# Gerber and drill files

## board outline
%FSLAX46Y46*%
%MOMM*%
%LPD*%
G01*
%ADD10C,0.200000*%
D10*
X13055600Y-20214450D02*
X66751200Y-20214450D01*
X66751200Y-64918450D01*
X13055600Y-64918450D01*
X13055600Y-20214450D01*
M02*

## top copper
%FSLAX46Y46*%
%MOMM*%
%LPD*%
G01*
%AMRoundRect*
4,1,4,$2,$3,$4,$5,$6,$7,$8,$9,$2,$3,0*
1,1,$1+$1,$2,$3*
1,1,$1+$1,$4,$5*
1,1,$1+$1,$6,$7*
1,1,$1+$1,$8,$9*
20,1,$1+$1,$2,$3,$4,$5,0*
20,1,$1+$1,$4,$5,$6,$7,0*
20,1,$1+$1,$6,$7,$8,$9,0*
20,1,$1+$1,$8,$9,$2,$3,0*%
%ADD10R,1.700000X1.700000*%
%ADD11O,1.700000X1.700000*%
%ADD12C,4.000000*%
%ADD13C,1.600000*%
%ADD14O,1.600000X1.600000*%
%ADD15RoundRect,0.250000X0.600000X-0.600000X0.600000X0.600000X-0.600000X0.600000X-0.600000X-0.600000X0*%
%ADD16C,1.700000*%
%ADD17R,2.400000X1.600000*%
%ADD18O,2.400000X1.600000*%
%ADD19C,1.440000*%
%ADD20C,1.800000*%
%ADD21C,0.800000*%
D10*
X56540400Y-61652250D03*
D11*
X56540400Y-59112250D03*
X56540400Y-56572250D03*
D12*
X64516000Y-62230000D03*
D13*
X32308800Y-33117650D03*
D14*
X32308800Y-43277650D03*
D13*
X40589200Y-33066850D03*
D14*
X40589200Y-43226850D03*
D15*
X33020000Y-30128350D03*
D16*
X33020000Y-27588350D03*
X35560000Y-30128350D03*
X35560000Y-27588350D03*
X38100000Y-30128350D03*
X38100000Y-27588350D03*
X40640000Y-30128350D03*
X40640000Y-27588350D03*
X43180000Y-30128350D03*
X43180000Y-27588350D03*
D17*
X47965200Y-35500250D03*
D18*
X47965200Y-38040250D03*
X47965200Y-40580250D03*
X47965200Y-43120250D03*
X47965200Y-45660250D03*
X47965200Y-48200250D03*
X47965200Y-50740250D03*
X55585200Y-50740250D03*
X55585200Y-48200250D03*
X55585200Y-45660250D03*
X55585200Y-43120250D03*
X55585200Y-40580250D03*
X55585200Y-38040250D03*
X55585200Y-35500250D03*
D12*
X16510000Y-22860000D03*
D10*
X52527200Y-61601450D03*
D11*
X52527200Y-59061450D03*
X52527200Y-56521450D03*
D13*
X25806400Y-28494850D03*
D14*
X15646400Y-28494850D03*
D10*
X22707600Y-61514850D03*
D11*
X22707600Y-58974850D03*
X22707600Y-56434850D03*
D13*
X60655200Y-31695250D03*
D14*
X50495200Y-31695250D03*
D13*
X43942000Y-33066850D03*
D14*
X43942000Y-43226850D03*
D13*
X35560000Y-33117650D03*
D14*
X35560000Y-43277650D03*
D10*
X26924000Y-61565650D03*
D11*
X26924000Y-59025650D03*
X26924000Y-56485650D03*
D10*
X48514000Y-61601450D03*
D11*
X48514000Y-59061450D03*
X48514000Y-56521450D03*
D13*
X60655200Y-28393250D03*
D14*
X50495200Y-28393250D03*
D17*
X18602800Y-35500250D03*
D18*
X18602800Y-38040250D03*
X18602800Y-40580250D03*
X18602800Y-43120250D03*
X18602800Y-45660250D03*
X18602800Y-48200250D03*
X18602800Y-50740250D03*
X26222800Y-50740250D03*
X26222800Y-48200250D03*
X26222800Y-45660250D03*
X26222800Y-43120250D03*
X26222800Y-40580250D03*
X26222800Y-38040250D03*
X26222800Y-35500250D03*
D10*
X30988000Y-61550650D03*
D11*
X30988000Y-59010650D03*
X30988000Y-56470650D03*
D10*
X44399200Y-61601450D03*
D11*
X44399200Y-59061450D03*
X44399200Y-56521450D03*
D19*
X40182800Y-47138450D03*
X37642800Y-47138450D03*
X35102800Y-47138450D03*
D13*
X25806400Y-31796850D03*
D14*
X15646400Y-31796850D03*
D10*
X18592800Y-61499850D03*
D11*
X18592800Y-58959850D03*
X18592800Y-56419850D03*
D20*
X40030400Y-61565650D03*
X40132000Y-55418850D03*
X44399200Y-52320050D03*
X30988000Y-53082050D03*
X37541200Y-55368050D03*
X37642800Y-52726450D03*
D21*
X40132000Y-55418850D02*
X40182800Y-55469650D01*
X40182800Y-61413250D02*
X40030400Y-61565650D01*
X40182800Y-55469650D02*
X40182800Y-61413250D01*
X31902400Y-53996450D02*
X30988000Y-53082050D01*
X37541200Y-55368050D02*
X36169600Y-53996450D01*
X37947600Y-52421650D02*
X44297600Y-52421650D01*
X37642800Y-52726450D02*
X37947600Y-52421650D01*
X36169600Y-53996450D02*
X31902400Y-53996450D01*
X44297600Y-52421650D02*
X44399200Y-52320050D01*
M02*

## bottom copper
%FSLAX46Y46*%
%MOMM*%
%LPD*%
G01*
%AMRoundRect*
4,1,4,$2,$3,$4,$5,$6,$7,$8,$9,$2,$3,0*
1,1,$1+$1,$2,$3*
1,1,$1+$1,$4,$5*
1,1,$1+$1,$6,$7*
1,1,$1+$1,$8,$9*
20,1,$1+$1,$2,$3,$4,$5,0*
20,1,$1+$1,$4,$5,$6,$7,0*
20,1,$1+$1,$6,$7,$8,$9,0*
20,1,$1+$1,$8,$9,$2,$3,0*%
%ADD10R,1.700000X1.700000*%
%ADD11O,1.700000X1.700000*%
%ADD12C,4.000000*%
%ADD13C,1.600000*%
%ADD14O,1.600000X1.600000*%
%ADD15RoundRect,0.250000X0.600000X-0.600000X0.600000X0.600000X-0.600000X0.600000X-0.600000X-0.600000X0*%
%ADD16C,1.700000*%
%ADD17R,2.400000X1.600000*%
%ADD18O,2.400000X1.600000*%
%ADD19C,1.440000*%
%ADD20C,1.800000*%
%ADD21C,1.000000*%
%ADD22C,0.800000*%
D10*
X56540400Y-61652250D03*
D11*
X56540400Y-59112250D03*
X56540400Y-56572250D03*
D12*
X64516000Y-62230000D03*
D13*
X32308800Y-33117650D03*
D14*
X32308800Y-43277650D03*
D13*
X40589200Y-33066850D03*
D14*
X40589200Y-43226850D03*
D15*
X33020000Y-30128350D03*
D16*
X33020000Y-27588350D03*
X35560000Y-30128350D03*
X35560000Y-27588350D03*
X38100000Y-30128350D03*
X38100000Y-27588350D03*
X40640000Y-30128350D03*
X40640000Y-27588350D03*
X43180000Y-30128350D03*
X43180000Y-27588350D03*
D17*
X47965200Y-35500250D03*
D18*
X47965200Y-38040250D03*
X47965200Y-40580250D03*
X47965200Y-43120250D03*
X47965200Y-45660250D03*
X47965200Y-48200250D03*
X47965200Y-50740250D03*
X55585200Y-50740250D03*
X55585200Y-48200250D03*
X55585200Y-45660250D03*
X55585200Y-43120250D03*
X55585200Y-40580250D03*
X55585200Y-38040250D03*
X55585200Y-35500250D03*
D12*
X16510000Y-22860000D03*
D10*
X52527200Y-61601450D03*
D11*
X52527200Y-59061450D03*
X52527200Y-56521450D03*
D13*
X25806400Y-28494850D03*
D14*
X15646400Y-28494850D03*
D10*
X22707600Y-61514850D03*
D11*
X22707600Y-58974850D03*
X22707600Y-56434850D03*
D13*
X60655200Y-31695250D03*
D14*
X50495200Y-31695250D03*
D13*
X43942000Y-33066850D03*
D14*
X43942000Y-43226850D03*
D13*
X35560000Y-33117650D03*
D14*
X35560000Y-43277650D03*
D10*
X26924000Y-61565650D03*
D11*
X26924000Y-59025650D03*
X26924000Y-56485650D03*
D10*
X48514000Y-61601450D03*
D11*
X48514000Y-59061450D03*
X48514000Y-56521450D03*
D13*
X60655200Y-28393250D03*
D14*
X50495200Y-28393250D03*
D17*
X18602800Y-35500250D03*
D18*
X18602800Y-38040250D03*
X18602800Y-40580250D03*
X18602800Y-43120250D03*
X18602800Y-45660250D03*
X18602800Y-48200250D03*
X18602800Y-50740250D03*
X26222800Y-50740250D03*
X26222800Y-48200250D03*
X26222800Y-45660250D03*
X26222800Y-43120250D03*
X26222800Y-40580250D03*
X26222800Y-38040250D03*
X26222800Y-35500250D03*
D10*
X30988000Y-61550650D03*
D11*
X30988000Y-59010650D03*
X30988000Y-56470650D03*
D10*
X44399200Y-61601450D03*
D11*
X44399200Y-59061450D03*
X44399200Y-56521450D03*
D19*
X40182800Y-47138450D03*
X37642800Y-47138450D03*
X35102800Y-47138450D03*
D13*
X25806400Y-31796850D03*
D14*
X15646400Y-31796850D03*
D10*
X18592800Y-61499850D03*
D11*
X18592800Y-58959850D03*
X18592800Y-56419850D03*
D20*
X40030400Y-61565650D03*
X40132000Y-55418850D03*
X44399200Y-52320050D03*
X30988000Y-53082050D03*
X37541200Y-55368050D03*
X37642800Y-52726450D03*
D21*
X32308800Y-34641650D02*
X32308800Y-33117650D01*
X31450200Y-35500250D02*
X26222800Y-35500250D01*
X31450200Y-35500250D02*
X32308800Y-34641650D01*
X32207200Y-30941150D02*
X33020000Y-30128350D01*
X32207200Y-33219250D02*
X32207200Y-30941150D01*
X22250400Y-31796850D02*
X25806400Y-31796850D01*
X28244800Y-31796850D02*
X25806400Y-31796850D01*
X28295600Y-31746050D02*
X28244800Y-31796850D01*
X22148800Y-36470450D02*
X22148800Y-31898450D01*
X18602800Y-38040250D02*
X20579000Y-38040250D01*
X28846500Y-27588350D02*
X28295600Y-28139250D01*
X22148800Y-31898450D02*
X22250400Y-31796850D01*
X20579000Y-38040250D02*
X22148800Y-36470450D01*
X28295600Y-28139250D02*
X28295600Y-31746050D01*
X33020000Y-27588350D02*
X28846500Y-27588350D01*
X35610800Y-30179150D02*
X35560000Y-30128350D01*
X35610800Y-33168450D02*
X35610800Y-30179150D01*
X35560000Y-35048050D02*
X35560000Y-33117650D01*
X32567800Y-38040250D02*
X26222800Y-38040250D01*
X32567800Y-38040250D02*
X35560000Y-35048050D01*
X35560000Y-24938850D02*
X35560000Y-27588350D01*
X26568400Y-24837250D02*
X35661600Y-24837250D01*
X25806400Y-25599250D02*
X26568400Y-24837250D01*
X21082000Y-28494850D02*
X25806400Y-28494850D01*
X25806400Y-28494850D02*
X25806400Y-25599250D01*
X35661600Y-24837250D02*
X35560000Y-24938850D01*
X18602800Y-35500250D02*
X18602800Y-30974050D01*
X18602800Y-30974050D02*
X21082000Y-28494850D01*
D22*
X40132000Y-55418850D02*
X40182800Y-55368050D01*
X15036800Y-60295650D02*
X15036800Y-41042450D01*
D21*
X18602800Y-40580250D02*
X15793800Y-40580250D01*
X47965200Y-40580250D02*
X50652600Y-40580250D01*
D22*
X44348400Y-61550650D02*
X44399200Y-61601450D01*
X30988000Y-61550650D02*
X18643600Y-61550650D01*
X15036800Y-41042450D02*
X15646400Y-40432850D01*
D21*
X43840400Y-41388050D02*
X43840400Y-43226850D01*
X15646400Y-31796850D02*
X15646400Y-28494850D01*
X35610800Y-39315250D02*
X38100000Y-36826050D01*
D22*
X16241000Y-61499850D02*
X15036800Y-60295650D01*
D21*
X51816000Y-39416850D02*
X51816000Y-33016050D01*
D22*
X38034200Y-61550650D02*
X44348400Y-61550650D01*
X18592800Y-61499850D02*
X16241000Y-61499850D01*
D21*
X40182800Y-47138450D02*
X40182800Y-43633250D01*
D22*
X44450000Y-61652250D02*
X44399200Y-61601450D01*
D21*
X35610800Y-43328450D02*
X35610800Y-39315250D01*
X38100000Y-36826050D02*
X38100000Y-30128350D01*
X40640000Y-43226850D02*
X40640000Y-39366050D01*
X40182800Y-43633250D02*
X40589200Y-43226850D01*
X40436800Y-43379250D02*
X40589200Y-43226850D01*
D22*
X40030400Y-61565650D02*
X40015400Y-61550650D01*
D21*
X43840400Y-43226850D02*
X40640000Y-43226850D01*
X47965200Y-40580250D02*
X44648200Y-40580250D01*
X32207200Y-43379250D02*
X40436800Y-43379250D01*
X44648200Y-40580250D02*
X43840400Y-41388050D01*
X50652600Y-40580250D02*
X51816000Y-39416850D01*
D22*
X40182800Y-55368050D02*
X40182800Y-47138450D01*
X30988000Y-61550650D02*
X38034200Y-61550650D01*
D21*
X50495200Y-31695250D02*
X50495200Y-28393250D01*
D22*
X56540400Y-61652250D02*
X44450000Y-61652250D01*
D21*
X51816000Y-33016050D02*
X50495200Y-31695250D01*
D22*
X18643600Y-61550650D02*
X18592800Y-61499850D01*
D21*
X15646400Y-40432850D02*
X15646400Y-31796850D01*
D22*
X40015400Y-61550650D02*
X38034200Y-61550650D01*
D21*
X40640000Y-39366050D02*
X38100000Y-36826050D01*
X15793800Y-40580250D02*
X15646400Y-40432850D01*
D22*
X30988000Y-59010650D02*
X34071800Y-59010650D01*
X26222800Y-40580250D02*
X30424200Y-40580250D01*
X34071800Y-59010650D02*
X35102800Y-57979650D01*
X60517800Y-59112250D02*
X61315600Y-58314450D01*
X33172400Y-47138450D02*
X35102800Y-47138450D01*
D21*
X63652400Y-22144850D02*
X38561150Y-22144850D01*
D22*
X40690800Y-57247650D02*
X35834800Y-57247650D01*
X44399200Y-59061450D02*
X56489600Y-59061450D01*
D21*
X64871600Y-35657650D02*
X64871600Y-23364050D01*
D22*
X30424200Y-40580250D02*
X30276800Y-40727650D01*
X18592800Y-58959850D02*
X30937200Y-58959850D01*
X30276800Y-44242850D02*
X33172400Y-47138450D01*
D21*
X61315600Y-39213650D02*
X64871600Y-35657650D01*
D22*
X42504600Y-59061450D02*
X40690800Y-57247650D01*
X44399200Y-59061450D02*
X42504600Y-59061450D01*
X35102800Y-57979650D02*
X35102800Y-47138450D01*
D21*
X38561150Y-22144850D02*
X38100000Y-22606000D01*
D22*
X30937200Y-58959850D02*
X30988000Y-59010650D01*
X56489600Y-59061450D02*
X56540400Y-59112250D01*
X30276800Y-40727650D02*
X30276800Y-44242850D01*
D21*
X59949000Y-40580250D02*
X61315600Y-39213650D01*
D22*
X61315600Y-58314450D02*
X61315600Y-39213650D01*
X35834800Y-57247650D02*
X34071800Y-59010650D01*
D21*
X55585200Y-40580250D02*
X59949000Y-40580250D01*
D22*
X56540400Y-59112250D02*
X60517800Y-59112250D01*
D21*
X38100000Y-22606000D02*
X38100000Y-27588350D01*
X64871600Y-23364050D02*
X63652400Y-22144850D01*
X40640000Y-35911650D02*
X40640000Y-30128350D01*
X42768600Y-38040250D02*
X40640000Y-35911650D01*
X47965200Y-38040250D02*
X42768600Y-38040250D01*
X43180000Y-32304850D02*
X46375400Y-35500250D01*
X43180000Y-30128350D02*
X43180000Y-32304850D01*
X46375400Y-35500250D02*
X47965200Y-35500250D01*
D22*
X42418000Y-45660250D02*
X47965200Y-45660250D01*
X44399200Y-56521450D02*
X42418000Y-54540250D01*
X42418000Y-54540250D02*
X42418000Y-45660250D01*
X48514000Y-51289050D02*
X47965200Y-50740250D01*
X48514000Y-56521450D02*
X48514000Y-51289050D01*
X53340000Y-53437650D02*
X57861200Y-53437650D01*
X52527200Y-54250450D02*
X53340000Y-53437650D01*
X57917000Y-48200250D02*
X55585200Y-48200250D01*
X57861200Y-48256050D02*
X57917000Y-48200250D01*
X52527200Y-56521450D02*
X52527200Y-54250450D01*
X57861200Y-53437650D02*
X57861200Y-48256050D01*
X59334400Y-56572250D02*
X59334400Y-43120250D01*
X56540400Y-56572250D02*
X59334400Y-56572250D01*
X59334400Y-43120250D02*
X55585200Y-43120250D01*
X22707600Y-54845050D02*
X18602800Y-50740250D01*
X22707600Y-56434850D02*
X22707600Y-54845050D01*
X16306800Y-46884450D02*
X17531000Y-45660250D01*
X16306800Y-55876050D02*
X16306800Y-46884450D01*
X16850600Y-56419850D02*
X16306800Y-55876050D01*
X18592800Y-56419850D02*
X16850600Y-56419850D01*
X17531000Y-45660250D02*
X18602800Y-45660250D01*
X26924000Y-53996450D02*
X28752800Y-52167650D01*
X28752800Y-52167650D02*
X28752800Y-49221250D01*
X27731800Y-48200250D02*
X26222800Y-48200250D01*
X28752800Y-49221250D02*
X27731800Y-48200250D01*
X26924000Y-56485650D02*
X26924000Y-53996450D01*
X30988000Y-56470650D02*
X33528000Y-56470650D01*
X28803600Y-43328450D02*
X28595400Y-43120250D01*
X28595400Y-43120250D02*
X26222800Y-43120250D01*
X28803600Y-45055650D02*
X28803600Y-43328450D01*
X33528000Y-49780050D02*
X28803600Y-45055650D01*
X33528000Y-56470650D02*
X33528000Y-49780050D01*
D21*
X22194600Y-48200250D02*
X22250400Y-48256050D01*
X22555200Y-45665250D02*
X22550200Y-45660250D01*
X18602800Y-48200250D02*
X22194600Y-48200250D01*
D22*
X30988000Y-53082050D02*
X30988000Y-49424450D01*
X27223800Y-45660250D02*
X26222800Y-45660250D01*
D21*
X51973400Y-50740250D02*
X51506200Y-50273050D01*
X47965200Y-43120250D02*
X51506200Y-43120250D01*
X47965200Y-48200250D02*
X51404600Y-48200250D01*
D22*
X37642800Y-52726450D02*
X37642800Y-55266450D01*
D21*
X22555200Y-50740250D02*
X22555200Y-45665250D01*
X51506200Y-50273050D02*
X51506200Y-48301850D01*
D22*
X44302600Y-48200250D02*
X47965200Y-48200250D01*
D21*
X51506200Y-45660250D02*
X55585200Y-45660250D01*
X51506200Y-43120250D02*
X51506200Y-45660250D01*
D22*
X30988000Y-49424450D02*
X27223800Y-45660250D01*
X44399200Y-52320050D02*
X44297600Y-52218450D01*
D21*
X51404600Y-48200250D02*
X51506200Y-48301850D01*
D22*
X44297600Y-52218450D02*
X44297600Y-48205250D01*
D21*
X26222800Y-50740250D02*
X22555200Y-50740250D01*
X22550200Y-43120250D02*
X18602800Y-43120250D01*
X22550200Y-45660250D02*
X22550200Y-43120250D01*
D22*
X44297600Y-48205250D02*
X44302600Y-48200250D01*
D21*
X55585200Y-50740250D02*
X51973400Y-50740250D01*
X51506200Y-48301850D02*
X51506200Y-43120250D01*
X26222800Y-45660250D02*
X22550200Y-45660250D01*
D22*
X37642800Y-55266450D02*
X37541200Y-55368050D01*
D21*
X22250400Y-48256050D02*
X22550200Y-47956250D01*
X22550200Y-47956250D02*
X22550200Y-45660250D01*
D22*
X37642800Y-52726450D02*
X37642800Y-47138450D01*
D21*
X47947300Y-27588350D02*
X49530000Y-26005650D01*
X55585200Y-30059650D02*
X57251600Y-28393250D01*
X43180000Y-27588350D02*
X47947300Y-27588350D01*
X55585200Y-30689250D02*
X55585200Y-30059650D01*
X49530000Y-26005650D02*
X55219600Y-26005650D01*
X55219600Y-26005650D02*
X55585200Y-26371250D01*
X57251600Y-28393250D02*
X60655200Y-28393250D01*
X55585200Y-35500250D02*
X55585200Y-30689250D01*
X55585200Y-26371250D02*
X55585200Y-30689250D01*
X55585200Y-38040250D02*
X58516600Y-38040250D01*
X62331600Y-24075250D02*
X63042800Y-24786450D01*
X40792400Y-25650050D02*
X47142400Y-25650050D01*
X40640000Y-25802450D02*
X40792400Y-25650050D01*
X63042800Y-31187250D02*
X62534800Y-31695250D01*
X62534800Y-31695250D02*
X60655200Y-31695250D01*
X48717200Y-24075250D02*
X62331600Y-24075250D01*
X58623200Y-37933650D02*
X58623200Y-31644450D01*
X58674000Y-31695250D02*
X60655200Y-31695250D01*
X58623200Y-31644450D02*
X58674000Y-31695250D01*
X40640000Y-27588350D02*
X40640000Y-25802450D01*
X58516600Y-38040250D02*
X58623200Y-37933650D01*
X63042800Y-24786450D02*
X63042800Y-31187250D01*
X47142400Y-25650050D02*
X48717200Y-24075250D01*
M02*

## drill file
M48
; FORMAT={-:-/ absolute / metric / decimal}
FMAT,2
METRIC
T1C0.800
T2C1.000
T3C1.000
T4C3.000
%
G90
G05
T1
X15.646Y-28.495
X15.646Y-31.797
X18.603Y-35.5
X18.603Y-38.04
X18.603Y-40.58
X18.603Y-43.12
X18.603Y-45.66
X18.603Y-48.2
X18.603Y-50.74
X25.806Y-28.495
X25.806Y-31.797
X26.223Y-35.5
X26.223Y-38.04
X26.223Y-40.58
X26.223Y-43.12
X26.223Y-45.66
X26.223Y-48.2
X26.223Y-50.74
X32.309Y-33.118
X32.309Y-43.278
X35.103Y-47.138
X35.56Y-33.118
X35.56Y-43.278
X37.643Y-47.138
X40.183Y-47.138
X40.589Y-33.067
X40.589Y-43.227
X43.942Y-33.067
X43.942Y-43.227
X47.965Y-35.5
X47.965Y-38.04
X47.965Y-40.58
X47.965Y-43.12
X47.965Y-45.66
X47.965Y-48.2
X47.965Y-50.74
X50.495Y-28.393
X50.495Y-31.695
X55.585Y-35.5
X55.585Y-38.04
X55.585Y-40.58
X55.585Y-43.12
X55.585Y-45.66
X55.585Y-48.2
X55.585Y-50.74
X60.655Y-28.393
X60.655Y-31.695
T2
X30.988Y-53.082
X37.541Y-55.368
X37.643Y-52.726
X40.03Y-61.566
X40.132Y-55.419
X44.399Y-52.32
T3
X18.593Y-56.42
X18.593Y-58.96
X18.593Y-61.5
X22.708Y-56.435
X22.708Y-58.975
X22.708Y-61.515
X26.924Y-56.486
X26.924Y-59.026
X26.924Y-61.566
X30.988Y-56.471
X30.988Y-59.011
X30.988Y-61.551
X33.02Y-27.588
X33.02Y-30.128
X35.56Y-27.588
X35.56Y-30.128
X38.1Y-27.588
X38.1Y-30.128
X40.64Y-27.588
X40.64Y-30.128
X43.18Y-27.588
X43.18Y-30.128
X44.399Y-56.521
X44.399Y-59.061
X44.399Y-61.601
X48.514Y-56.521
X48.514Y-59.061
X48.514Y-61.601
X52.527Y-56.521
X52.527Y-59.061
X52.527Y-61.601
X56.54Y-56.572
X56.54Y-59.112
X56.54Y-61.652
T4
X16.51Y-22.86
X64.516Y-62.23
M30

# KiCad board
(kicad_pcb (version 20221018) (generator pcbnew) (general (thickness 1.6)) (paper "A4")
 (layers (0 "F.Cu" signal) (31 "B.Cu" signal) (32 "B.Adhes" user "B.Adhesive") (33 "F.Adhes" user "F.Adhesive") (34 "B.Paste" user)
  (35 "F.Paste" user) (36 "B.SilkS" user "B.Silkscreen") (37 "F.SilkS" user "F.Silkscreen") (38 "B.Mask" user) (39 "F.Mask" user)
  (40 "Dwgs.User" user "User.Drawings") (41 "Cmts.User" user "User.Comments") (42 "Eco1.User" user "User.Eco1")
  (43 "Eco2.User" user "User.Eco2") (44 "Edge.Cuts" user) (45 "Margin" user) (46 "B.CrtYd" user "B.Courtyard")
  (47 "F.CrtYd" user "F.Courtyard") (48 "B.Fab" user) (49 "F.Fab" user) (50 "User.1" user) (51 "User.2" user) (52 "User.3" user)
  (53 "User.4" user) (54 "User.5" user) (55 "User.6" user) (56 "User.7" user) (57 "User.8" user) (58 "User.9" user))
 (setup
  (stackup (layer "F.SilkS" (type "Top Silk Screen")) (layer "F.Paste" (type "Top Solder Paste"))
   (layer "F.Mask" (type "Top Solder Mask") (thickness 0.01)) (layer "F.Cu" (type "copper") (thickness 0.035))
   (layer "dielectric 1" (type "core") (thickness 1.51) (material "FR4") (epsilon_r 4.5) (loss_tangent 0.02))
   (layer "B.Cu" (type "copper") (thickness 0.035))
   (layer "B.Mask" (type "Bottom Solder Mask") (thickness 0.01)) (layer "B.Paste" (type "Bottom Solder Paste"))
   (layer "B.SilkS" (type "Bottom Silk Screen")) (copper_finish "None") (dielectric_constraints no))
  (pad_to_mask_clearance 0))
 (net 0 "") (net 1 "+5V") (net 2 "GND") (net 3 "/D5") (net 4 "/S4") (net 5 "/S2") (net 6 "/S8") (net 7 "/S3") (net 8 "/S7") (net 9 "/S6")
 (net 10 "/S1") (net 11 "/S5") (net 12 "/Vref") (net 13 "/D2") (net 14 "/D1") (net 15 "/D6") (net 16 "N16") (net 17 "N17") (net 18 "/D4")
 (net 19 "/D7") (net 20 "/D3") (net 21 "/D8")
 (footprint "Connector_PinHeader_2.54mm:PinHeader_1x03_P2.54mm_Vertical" (layer "F.Cu") (at 56.5404 61.65225 180)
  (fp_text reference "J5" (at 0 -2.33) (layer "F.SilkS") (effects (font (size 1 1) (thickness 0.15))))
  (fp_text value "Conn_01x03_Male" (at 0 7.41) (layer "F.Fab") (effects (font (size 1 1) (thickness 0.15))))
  (pad "1" thru_hole rect (at 0 0 180) (size 1.7 1.7) (drill 1) (layers "*.Cu" "*.Mask") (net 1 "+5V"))
  (pad "2" thru_hole oval (at 0 2.54 180) (size 1.7 1.7) (drill 1) (layers "*.Cu" "*.Mask") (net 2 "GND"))
  (pad "3" thru_hole oval (at 0 5.08 180) (size 1.7 1.7) (drill 1) (layers "*.Cu" "*.Mask") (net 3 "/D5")))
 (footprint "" (layer "F.Cu") (at 64.516 62.23)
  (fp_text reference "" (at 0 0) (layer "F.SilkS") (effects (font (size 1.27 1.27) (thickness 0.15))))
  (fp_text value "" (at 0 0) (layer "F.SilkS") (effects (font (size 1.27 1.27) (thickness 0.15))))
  (pad "1" thru_hole circle (at 0 0) (size 4 4) (drill 3) (layers "*.Cu" "*.Mask")))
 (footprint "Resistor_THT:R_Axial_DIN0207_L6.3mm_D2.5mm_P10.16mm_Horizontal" (layer "F.Cu") (at 32.3088 33.11765 -90)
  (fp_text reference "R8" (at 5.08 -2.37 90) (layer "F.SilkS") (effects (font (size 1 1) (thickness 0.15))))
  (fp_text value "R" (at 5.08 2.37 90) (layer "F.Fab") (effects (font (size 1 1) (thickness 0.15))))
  (pad "1" thru_hole circle (at 0 0 270) (size 1.6 1.6) (drill 0.8) (layers "*.Cu" "*.Mask") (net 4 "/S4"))
  (pad "2" thru_hole oval (at 10.16 0 270) (size 1.6 1.6) (drill 0.8) (layers "*.Cu" "*.Mask") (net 1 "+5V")))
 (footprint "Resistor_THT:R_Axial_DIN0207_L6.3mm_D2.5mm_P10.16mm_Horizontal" (layer "F.Cu") (at 40.5892 33.06685 -90)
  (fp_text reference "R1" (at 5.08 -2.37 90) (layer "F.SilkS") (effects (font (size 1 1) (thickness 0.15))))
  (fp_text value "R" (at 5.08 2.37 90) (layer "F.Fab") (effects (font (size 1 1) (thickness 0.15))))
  (pad "1" thru_hole circle (at 0 0 270) (size 1.6 1.6) (drill 0.8) (layers "*.Cu" "*.Mask") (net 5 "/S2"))
  (pad "2" thru_hole oval (at 10.16 0 270) (size 1.6 1.6) (drill 0.8) (layers "*.Cu" "*.Mask") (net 1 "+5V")))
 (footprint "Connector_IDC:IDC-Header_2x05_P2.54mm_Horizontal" (layer "F.Cu") (at 33.02 30.12835 90)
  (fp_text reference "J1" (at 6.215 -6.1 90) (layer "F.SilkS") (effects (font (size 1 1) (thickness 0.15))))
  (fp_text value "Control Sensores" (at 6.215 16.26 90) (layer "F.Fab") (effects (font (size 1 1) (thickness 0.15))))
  (pad "1" thru_hole roundrect (at 0 0 90) (size 1.7 1.7) (drill 1) (layers "*.Cu" "*.Mask") (roundrect_rratio 0.147059) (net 4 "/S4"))
  (pad "2" thru_hole circle (at 2.54 0 90) (size 1.7 1.7) (drill 1) (layers "*.Cu" "*.Mask") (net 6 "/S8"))
  (pad "3" thru_hole circle (at 0 2.54 90) (size 1.7 1.7) (drill 1) (layers "*.Cu" "*.Mask") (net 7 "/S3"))
  (pad "4" thru_hole circle (at 2.54 2.54 90) (size 1.7 1.7) (drill 1) (layers "*.Cu" "*.Mask") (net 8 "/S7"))
  (pad "5" thru_hole circle (at 0 5.08 90) (size 1.7 1.7) (drill 1) (layers "*.Cu" "*.Mask") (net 1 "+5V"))
  (pad "6" thru_hole circle (at 2.54 5.08 90) (size 1.7 1.7) (drill 1) (layers "*.Cu" "*.Mask") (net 2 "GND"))
  (pad "7" thru_hole circle (at 0 7.62 90) (size 1.7 1.7) (drill 1) (layers "*.Cu" "*.Mask") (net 5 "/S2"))
  (pad "8" thru_hole circle (at 2.54 7.62 90) (size 1.7 1.7) (drill 1) (layers "*.Cu" "*.Mask") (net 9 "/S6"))
  (pad "9" thru_hole circle (at 0 10.16 90) (size 1.7 1.7) (drill 1) (layers "*.Cu" "*.Mask") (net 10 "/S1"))
  (pad "10" thru_hole circle (at 2.54 10.16 90) (size 1.7 1.7) (drill 1) (layers "*.Cu" "*.Mask") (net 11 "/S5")))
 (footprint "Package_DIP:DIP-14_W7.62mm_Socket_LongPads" (layer "F.Cu") (at 47.9652 35.50025)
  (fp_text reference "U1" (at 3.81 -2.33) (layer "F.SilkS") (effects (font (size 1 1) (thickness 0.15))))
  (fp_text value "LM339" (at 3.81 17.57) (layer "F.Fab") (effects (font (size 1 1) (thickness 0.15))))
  (pad "1" thru_hole rect (at 0 0) (size 2.4 1.6) (drill 0.8) (layers "*.Cu" "*.Mask") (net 10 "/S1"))
  (pad "2" thru_hole oval (at 0 2.54) (size 2.4 1.6) (drill 0.8) (layers "*.Cu" "*.Mask") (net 5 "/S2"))
  (pad "3" thru_hole oval (at 0 5.08) (size 2.4 1.6) (drill 0.8) (layers "*.Cu" "*.Mask") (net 1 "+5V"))
  (pad "4" thru_hole oval (at 0 7.62) (size 2.4 1.6) (drill 0.8) (layers "*.Cu" "*.Mask") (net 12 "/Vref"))
  (pad "5" thru_hole oval (at 0 10.16) (size 2.4 1.6) (drill 0.8) (layers "*.Cu" "*.Mask") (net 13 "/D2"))
  (pad "6" thru_hole oval (at 0 12.7) (size 2.4 1.6) (drill 0.8) (layers "*.Cu" "*.Mask") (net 12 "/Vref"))
  (pad "7" thru_hole oval (at 0 15.24) (size 2.4 1.6) (drill 0.8) (layers "*.Cu" "*.Mask") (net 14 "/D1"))
  (pad "8" thru_hole oval (at 7.62 15.24) (size 2.4 1.6) (drill 0.8) (layers "*.Cu" "*.Mask") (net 12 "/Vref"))
  (pad "9" thru_hole oval (at 7.62 12.7) (size 2.4 1.6) (drill 0.8) (layers "*.Cu" "*.Mask") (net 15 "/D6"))
  (pad "10" thru_hole oval (at 7.62 10.16) (size 2.4 1.6) (drill 0.8) (layers "*.Cu" "*.Mask") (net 12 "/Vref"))
  (pad "11" thru_hole oval (at 7.62 7.62) (size 2.4 1.6) (drill 0.8) (layers "*.Cu" "*.Mask") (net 3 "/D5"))
  (pad "12" thru_hole oval (at 7.62 5.08) (size 2.4 1.6) (drill 0.8) (layers "*.Cu" "*.Mask") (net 2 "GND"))
  (pad "13" thru_hole oval (at 7.62 2.54) (size 2.4 1.6) (drill 0.8) (layers "*.Cu" "*.Mask") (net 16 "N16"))
  (pad "14" thru_hole oval (at 7.62 0) (size 2.4 1.6) (drill 0.8) (layers "*.Cu" "*.Mask") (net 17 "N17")))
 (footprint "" (layer "F.Cu") (at 16.51 22.86)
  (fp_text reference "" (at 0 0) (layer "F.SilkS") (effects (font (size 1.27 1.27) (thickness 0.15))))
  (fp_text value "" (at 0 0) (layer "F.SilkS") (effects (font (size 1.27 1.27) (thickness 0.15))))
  (pad "1" thru_hole circle (at 0 0) (size 4 4) (drill 3) (layers "*.Cu" "*.Mask")))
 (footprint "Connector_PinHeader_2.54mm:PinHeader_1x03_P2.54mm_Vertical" (layer "F.Cu") (at 52.5272 61.60145 180)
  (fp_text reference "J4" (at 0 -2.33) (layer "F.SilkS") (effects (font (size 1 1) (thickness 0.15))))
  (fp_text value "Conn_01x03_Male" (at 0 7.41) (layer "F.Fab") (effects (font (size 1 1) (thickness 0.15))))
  (pad "1" thru_hole rect (at 0 0 180) (size 1.7 1.7) (drill 1) (layers "*.Cu" "*.Mask") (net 1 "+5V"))
  (pad "2" thru_hole oval (at 0 2.54 180) (size 1.7 1.7) (drill 1) (layers "*.Cu" "*.Mask") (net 2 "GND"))
  (pad "3" thru_hole oval (at 0 5.08 180) (size 1.7 1.7) (drill 1) (layers "*.Cu" "*.Mask") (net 15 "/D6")))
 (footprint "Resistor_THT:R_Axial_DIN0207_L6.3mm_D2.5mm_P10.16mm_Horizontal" (layer "F.Cu") (at 25.8064 28.49485 180)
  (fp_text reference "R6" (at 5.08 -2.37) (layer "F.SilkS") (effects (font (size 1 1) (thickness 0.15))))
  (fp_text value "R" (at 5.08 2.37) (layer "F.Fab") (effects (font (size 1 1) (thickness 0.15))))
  (pad "1" thru_hole circle (at 0 0 180) (size 1.6 1.6) (drill 0.8) (layers "*.Cu" "*.Mask") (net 8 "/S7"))
  (pad "2" thru_hole oval (at 10.16 0 180) (size 1.6 1.6) (drill 0.8) (layers "*.Cu" "*.Mask") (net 1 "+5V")))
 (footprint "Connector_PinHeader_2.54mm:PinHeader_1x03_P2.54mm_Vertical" (layer "F.Cu") (at 22.7076 61.51485 180)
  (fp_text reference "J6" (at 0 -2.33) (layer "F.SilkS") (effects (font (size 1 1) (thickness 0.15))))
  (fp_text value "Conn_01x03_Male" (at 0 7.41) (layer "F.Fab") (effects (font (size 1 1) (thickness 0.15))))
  (pad "1" thru_hole rect (at 0 0 180) (size 1.7 1.7) (drill 1) (layers "*.Cu" "*.Mask") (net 1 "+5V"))
  (pad "2" thru_hole oval (at 0 2.54 180) (size 1.7 1.7) (drill 1) (layers "*.Cu" "*.Mask") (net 2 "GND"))
  (pad "3" thru_hole oval (at 0 5.08 180) (size 1.7 1.7) (drill 1) (layers "*.Cu" "*.Mask") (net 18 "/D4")))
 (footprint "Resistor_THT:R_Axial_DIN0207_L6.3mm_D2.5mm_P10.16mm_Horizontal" (layer "F.Cu") (at 60.6552 31.69525 180)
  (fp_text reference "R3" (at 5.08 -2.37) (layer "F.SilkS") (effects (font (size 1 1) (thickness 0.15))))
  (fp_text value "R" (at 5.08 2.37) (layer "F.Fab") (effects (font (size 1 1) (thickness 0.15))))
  (pad "1" thru_hole circle (at 0 0 180) (size 1.6 1.6) (drill 0.8) (layers "*.Cu" "*.Mask") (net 16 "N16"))
  (pad "2" thru_hole oval (at 10.16 0 180) (size 1.6 1.6) (drill 0.8) (layers "*.Cu" "*.Mask") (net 1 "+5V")))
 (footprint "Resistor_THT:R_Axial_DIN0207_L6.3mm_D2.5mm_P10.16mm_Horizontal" (layer "F.Cu") (at 43.942 33.06685 -90)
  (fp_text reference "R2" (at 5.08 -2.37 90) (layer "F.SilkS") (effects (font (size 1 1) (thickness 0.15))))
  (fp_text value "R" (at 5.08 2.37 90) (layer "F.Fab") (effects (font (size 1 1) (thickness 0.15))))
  (pad "1" thru_hole circle (at 0 0 270) (size 1.6 1.6) (drill 0.8) (layers "*.Cu" "*.Mask") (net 10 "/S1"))
  (pad "2" thru_hole oval (at 10.16 0 270) (size 1.6 1.6) (drill 0.8) (layers "*.Cu" "*.Mask") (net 1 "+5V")))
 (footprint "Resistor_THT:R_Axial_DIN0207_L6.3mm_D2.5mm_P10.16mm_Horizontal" (layer "F.Cu") (at 35.56 33.11765 -90)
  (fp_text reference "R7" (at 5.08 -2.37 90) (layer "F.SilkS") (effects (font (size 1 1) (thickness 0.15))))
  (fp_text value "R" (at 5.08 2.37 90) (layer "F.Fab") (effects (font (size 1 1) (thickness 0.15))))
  (pad "1" thru_hole circle (at 0 0 270) (size 1.6 1.6) (drill 0.8) (layers "*.Cu" "*.Mask") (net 7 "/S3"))
  (pad "2" thru_hole oval (at 10.16 0 270) (size 1.6 1.6) (drill 0.8) (layers "*.Cu" "*.Mask") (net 1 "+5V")))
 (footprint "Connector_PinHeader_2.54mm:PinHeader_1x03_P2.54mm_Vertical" (layer "F.Cu") (at 26.924 61.56565 180)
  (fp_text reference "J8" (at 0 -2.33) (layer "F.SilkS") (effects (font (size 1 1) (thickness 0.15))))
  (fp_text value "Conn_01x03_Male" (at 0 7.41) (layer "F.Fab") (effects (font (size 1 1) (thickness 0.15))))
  (pad "1" thru_hole rect (at 0 0 180) (size 1.7 1.7) (drill 1) (layers "*.Cu" "*.Mask") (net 1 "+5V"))
  (pad "2" thru_hole oval (at 0 2.54 180) (size 1.7 1.7) (drill 1) (layers "*.Cu" "*.Mask") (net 2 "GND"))
  (pad "3" thru_hole oval (at 0 5.08 180) (size 1.7 1.7) (drill 1) (layers "*.Cu" "*.Mask") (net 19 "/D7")))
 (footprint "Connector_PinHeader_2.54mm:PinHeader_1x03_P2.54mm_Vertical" (layer "F.Cu") (at 48.514 61.60145 180)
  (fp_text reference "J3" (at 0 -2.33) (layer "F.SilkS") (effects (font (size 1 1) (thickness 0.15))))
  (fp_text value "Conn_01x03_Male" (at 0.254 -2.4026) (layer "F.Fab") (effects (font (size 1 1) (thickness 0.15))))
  (pad "1" thru_hole rect (at 0 0 180) (size 1.7 1.7) (drill 1) (layers "*.Cu" "*.Mask") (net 1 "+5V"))
  (pad "2" thru_hole oval (at 0 2.54 180) (size 1.7 1.7) (drill 1) (layers "*.Cu" "*.Mask") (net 2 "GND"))
  (pad "3" thru_hole oval (at 0 5.08 180) (size 1.7 1.7) (drill 1) (layers "*.Cu" "*.Mask") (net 14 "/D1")))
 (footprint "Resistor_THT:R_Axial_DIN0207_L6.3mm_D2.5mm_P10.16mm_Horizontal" (layer "F.Cu") (at 60.6552 28.39325 180)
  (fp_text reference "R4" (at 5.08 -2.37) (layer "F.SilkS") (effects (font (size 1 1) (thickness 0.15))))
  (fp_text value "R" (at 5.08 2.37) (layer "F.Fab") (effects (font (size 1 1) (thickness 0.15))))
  (pad "1" thru_hole circle (at 0 0 180) (size 1.6 1.6) (drill 0.8) (layers "*.Cu" "*.Mask") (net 17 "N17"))
  (pad "2" thru_hole oval (at 10.16 0 180) (size 1.6 1.6) (drill 0.8) (layers "*.Cu" "*.Mask") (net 1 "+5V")))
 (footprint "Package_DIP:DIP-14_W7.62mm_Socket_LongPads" (layer "F.Cu") (at 18.6028 35.50025)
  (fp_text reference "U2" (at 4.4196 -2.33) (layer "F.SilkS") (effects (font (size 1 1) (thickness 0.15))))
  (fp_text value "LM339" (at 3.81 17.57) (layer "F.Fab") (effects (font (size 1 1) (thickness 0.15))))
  (pad "1" thru_hole rect (at 0 0) (size 2.4 1.6) (drill 0.8) (layers "*.Cu" "*.Mask") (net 8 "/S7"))
  (pad "2" thru_hole oval (at 0 2.54) (size 2.4 1.6) (drill 0.8) (layers "*.Cu" "*.Mask") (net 6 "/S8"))
  (pad "3" thru_hole oval (at 0 5.08) (size 2.4 1.6) (drill 0.8) (layers "*.Cu" "*.Mask") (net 1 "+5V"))
  (pad "4" thru_hole oval (at 0 7.62) (size 2.4 1.6) (drill 0.8) (layers "*.Cu" "*.Mask") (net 12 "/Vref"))
  (pad "5" thru_hole oval (at 0 10.16) (size 2.4 1.6) (drill 0.8) (layers "*.Cu" "*.Mask") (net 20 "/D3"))
  (pad "6" thru_hole oval (at 0 12.7) (size 2.4 1.6) (drill 0.8) (layers "*.Cu" "*.Mask") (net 12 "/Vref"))
  (pad "7" thru_hole oval (at 0 15.24) (size 2.4 1.6) (drill 0.8) (layers "*.Cu" "*.Mask") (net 18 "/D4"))
  (pad "8" thru_hole oval (at 7.62 15.24) (size 2.4 1.6) (drill 0.8) (layers "*.Cu" "*.Mask") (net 12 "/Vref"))
  (pad "9" thru_hole oval (at 7.62 12.7) (size 2.4 1.6) (drill 0.8) (layers "*.Cu" "*.Mask") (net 19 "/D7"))
  (pad "10" thru_hole oval (at 7.62 10.16) (size 2.4 1.6) (drill 0.8) (layers "*.Cu" "*.Mask") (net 12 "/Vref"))
  (pad "11" thru_hole oval (at 7.62 7.62) (size 2.4 1.6) (drill 0.8) (layers "*.Cu" "*.Mask") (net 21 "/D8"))
  (pad "12" thru_hole oval (at 7.62 5.08) (size 2.4 1.6) (drill 0.8) (layers "*.Cu" "*.Mask") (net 2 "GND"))
  (pad "13" thru_hole oval (at 7.62 2.54) (size 2.4 1.6) (drill 0.8) (layers "*.Cu" "*.Mask") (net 7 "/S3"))
  (pad "14" thru_hole oval (at 7.62 0) (size 2.4 1.6) (drill 0.8) (layers "*.Cu" "*.Mask") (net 4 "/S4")))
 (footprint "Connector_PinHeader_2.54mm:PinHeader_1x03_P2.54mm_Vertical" (layer "F.Cu") (at 30.988 61.55065 180)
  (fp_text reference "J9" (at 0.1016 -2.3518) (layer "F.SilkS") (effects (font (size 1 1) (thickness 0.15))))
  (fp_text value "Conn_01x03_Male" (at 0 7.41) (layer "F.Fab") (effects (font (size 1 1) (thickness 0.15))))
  (pad "1" thru_hole rect (at 0 0 180) (size 1.7 1.7) (drill 1) (layers "*.Cu" "*.Mask") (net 1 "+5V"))
  (pad "2" thru_hole oval (at 0 2.54 180) (size 1.7 1.7) (drill 1) (layers "*.Cu" "*.Mask") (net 2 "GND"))
  (pad "3" thru_hole oval (at 0 5.08 180) (size 1.7 1.7) (drill 1) (layers "*.Cu" "*.Mask") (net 21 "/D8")))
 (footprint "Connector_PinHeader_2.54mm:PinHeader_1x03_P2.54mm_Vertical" (layer "F.Cu") (at 44.3992 61.60145 180)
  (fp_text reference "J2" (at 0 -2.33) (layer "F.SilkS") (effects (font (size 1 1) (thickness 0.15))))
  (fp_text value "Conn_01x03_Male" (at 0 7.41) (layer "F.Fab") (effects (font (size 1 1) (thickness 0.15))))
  (pad "1" thru_hole rect (at 0 0 180) (size 1.7 1.7) (drill 1) (layers "*.Cu" "*.Mask") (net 1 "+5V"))
  (pad "2" thru_hole oval (at 0 2.54 180) (size 1.7 1.7) (drill 1) (layers "*.Cu" "*.Mask") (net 2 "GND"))
  (pad "3" thru_hole oval (at 0 5.08 180) (size 1.7 1.7) (drill 1) (layers "*.Cu" "*.Mask") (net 13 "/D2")))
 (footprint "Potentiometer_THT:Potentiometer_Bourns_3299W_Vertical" (layer "F.Cu") (at 40.1828 47.13845)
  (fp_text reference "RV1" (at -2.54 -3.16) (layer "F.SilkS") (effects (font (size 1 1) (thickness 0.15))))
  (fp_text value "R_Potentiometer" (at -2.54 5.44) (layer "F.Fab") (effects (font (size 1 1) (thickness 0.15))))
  (pad "1" thru_hole circle (at 0 0) (size 1.44 1.44) (drill 0.8) (layers "*.Cu" "*.Mask") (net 1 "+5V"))
  (pad "2" thru_hole circle (at -2.54 0) (size 1.44 1.44) (drill 0.8) (layers "*.Cu" "*.Mask") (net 12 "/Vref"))
  (pad "3" thru_hole circle (at -5.08 0) (size 1.44 1.44) (drill 0.8) (layers "*.Cu" "*.Mask") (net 2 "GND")))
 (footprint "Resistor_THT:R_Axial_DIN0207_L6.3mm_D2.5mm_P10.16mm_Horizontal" (layer "F.Cu") (at 25.8064 31.79685 180)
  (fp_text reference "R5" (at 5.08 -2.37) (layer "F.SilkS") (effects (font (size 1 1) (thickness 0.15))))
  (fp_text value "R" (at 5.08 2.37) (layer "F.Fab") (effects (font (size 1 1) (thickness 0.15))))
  (pad "1" thru_hole circle (at 0 0 180) (size 1.6 1.6) (drill 0.8) (layers "*.Cu" "*.Mask") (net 6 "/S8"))
  (pad "2" thru_hole oval (at 10.16 0 180) (size 1.6 1.6) (drill 0.8) (layers "*.Cu" "*.Mask") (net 1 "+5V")))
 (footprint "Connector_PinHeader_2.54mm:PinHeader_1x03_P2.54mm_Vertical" (layer "F.Cu") (at 18.5928 61.49985 180)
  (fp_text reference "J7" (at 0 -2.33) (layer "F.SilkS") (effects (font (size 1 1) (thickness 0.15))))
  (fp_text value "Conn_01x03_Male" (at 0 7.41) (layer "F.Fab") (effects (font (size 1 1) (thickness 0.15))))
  (pad "1" thru_hole rect (at 0 0 180) (size 1.7 1.7) (drill 1) (layers "*.Cu" "*.Mask") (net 1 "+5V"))
  (pad "2" thru_hole oval (at 0 2.54 180) (size 1.7 1.7) (drill 1) (layers "*.Cu" "*.Mask") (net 2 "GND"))
  (pad "3" thru_hole oval (at 0 5.08 180) (size 1.7 1.7) (drill 1) (layers "*.Cu" "*.Mask") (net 20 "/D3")))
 (gr_rect (start 13.0556 20.21445) (end 66.7512 64.91845) (stroke (width 0.2) (type solid)) (fill none) (layer "Edge.Cuts"))
 (segment (start 32.3088 34.64165) (end 32.3088 33.11765) (width 1) (layer "B.Cu") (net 4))
 (segment (start 31.4502 35.50025) (end 26.2228 35.50025) (width 1) (layer "B.Cu") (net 4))
 (segment (start 31.4502 35.50025) (end 32.3088 34.64165) (width 1) (layer "B.Cu") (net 4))
 (segment (start 32.2072 30.94115) (end 33.02 30.12835) (width 1) (layer "B.Cu") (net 4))
 (segment (start 32.2072 33.21925) (end 32.2072 30.94115) (width 1) (layer "B.Cu") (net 4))
 (segment (start 22.2504 31.79685) (end 25.8064 31.79685) (width 1) (layer "B.Cu") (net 6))
 (segment (start 28.2448 31.79685) (end 25.8064 31.79685) (width 1) (layer "B.Cu") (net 6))
 (segment (start 28.2956 31.74605) (end 28.2448 31.79685) (width 1) (layer "B.Cu") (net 6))
 (segment (start 22.1488 36.47045) (end 22.1488 31.89845) (width 1) (layer "B.Cu") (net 6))
 (segment (start 18.6028 38.04025) (end 20.579 38.04025) (width 1) (layer "B.Cu") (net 6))
 (segment (start 28.8465 27.58835) (end 28.2956 28.13925) (width 1) (layer "B.Cu") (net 6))
 (segment (start 22.1488 31.89845) (end 22.2504 31.79685) (width 1) (layer "B.Cu") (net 6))
 (segment (start 20.579 38.04025) (end 22.1488 36.47045) (width 1) (layer "B.Cu") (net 6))
 (segment (start 28.2956 28.13925) (end 28.2956 31.74605) (width 1) (layer "B.Cu") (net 6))
 (segment (start 33.02 27.58835) (end 28.8465 27.58835) (width 1) (layer "B.Cu") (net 6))
 (segment (start 35.6108 30.17915) (end 35.56 30.12835) (width 1) (layer "B.Cu") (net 7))
 (segment (start 35.6108 33.16845) (end 35.6108 30.17915) (width 1) (layer "B.Cu") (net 7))
 (segment (start 35.56 35.04805) (end 35.56 33.11765) (width 1) (layer "B.Cu") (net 7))
 (segment (start 32.5678 38.04025) (end 26.2228 38.04025) (width 1) (layer "B.Cu") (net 7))
 (segment (start 32.5678 38.04025) (end 35.56 35.04805) (width 1) (layer "B.Cu") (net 7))
 (segment (start 35.56 24.93885) (end 35.56 27.58835) (width 1) (layer "B.Cu") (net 8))
 (segment (start 26.5684 24.83725) (end 35.6616 24.83725) (width 1) (layer "B.Cu") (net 8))
 (segment (start 25.8064 25.59925) (end 26.5684 24.83725) (width 1) (layer "B.Cu") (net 8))
 (segment (start 21.082 28.49485) (end 25.8064 28.49485) (width 1) (layer "B.Cu") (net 8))
 (segment (start 25.8064 28.49485) (end 25.8064 25.59925) (width 1) (layer "B.Cu") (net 8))
 (segment (start 35.6616 24.83725) (end 35.56 24.93885) (width 1) (layer "B.Cu") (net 8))
 (segment (start 18.6028 35.50025) (end 18.6028 30.97405) (width 1) (layer "B.Cu") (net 8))
 (segment (start 18.6028 30.97405) (end 21.082 28.49485) (width 1) (layer "B.Cu") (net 8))
 (segment (start 40.132 55.41885) (end 40.1828 55.46965) (width 0.8) (layer "F.Cu") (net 1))
 (segment (start 40.1828 61.41325) (end 40.0304 61.56565) (width 0.8) (layer "F.Cu") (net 1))
 (segment (start 40.1828 55.46965) (end 40.1828 61.41325) (width 0.8) (layer "F.Cu") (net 1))
 (via (at 40.0304 61.56565) (size 1.8) (drill 1) (layers "F.Cu" "B.Cu") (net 1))
 (via (at 40.132 55.41885) (size 1.8) (drill 1) (layers "F.Cu" "B.Cu") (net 1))
 (segment (start 40.132 55.41885) (end 40.1828 55.36805) (width 0.8) (layer "B.Cu") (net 1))
 (segment (start 15.0368 60.29565) (end 15.0368 41.04245) (width 0.8) (layer "B.Cu") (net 1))
 (segment (start 18.6028 40.58025) (end 15.7938 40.58025) (width 1) (layer "B.Cu") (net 1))
 (segment (start 47.9652 40.58025) (end 50.6526 40.58025) (width 1) (layer "B.Cu") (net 1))
 (segment (start 44.3484 61.55065) (end 44.3992 61.60145) (width 0.8) (layer "B.Cu") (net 1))
 (segment (start 30.988 61.55065) (end 18.6436 61.55065) (width 0.8) (layer "B.Cu") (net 1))
 (segment (start 15.0368 41.04245) (end 15.6464 40.43285) (width 0.8) (layer "B.Cu") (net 1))
 (segment (start 43.8404 41.38805) (end 43.8404 43.22685) (width 1) (layer "B.Cu") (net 1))
 (segment (start 15.6464 31.79685) (end 15.6464 28.49485) (width 1) (layer "B.Cu") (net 1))
 (segment (start 35.6108 39.31525) (end 38.1 36.82605) (width 1) (layer "B.Cu") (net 1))
 (segment (start 16.241 61.49985) (end 15.0368 60.29565) (width 0.8) (layer "B.Cu") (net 1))
 (segment (start 51.816 39.41685) (end 51.816 33.01605) (width 1) (layer "B.Cu") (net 1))
 (segment (start 38.0342 61.55065) (end 44.3484 61.55065) (width 0.8) (layer "B.Cu") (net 1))
 (segment (start 18.5928 61.49985) (end 16.241 61.49985) (width 0.8) (layer "B.Cu") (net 1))
 (segment (start 40.1828 47.13845) (end 40.1828 43.63325) (width 1) (layer "B.Cu") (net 1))
 (segment (start 44.45 61.65225) (end 44.3992 61.60145) (width 0.8) (layer "B.Cu") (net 1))
 (segment (start 35.6108 43.32845) (end 35.6108 39.31525) (width 1) (layer "B.Cu") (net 1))
 (segment (start 38.1 36.82605) (end 38.1 30.12835) (width 1) (layer "B.Cu") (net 1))
 (segment (start 40.64 43.22685) (end 40.64 39.36605) (width 1) (layer "B.Cu") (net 1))
 (segment (start 40.1828 43.63325) (end 40.5892 43.22685) (width 1) (layer "B.Cu") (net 1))
 (segment (start 40.4368 43.37925) (end 40.5892 43.22685) (width 1) (layer "B.Cu") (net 1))
 (segment (start 40.0304 61.56565) (end 40.0154 61.55065) (width 0.8) (layer "B.Cu") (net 1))
 (segment (start 43.8404 43.22685) (end 40.64 43.22685) (width 1) (layer "B.Cu") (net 1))
 (segment (start 47.9652 40.58025) (end 44.6482 40.58025) (width 1) (layer "B.Cu") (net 1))
 (segment (start 32.2072 43.37925) (end 40.4368 43.37925) (width 1) (layer "B.Cu") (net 1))
 (segment (start 44.6482 40.58025) (end 43.8404 41.38805) (width 1) (layer "B.Cu") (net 1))
 (segment (start 50.6526 40.58025) (end 51.816 39.41685) (width 1) (layer "B.Cu") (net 1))
 (segment (start 40.1828 55.36805) (end 40.1828 47.13845) (width 0.8) (layer "B.Cu") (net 1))
 (segment (start 30.988 61.55065) (end 38.0342 61.55065) (width 0.8) (layer "B.Cu") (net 1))
 (segment (start 50.4952 31.69525) (end 50.4952 28.39325) (width 1) (layer "B.Cu") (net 1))
 (segment (start 56.5404 61.65225) (end 44.45 61.65225) (width 0.8) (layer "B.Cu") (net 1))
 (segment (start 51.816 33.01605) (end 50.4952 31.69525) (width 1) (layer "B.Cu") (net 1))
 (segment (start 18.6436 61.55065) (end 18.5928 61.49985) (width 0.8) (layer "B.Cu") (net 1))
 (segment (start 15.6464 40.43285) (end 15.6464 31.79685) (width 1) (layer "B.Cu") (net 1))
 (segment (start 40.0154 61.55065) (end 38.0342 61.55065) (width 0.8) (layer "B.Cu") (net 1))
 (segment (start 40.64 39.36605) (end 38.1 36.82605) (width 1) (layer "B.Cu") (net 1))
 (segment (start 15.7938 40.58025) (end 15.6464 40.43285) (width 1) (layer "B.Cu") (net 1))
 (segment (start 30.988 59.01065) (end 34.0718 59.01065) (width 0.8) (layer "B.Cu") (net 2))
 (segment (start 26.2228 40.58025) (end 30.4242 40.58025) (width 0.8) (layer "B.Cu") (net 2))
 (segment (start 34.0718 59.01065) (end 35.1028 57.97965) (width 0.8) (layer "B.Cu") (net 2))
 (segment (start 60.5178 59.11225) (end 61.3156 58.31445) (width 0.8) (layer "B.Cu") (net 2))
 (segment (start 33.1724 47.13845) (end 35.1028 47.13845) (width 0.8) (layer "B.Cu") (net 2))
 (segment (start 63.6524 22.14485) (end 38.56115 22.14485) (width 1) (layer "B.Cu") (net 2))
 (segment (start 40.6908 57.24765) (end 35.8348 57.24765) (width 0.8) (layer "B.Cu") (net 2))
 (segment (start 44.3992 59.06145) (end 56.4896 59.06145) (width 0.8) (layer "B.Cu") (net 2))
 (segment (start 64.8716 35.65765) (end 64.8716 23.36405) (width 1) (layer "B.Cu") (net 2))
 (segment (start 30.4242 40.58025) (end 30.2768 40.72765) (width 0.8) (layer "B.Cu") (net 2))
 (segment (start 18.5928 58.95985) (end 30.9372 58.95985) (width 0.8) (layer "B.Cu") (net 2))
 (segment (start 30.2768 44.24285) (end 33.1724 47.13845) (width 0.8) (layer "B.Cu") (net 2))
 (segment (start 61.3156 39.21365) (end 64.8716 35.65765) (width 1) (layer "B.Cu") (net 2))
 (segment (start 42.5046 59.06145) (end 40.6908 57.24765) (width 0.8) (layer "B.Cu") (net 2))
 (segment (start 44.3992 59.06145) (end 42.5046 59.06145) (width 0.8) (layer "B.Cu") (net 2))
 (segment (start 35.1028 57.97965) (end 35.1028 47.13845) (width 0.8) (layer "B.Cu") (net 2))
 (segment (start 38.56115 22.14485) (end 38.1 22.606) (width 1) (layer "B.Cu") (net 2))
 (segment (start 30.9372 58.95985) (end 30.988 59.01065) (width 0.8) (layer "B.Cu") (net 2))
 (segment (start 56.4896 59.06145) (end 56.5404 59.11225) (width 0.8) (layer "B.Cu") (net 2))
 (segment (start 30.2768 40.72765) (end 30.2768 44.24285) (width 0.8) (layer "B.Cu") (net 2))
 (segment (start 59.949 40.58025) (end 61.3156 39.21365) (width 1) (layer "B.Cu") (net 2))
 (segment (start 61.3156 58.31445) (end 61.3156 39.21365) (width 0.8) (layer "B.Cu") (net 2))
 (segment (start 35.8348 57.24765) (end 34.0718 59.01065) (width 0.8) (layer "B.Cu") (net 2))
 (segment (start 55.5852 40.58025) (end 59.949 40.58025) (width 1) (layer "B.Cu") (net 2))
 (segment (start 56.5404 59.11225) (end 60.5178 59.11225) (width 0.8) (layer "B.Cu") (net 2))
 (segment (start 38.1 22.606) (end 38.1 27.58835) (width 1) (layer "B.Cu") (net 2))
 (segment (start 64.8716 23.36405) (end 63.6524 22.14485) (width 1) (layer "B.Cu") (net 2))
 (segment (start 40.64 35.91165) (end 40.64 30.12835) (width 1) (layer "B.Cu") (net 5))
 (segment (start 42.7686 38.04025) (end 40.64 35.91165) (width 1) (layer "B.Cu") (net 5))
 (segment (start 47.9652 38.04025) (end 42.7686 38.04025) (width 1) (layer "B.Cu") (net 5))
 (segment (start 43.18 32.30485) (end 46.3754 35.50025) (width 1) (layer "B.Cu") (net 10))
 (segment (start 43.18 30.12835) (end 43.18 32.30485) (width 1) (layer "B.Cu") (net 10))
 (segment (start 46.3754 35.50025) (end 47.9652 35.50025) (width 1) (layer "B.Cu") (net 10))
 (segment (start 42.418 45.66025) (end 47.9652 45.66025) (width 0.8) (layer "B.Cu") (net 13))
 (segment (start 44.3992 56.52145) (end 42.418 54.54025) (width 0.8) (layer "B.Cu") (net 13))
 (segment (start 42.418 54.54025) (end 42.418 45.66025) (width 0.8) (layer "B.Cu") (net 13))
 (segment (start 48.514 51.28905) (end 47.9652 50.74025) (width 0.8) (layer "B.Cu") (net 14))
 (segment (start 48.514 56.52145) (end 48.514 51.28905) (width 0.8) (layer "B.Cu") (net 14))
 (segment (start 53.34 53.43765) (end 57.8612 53.43765) (width 0.8) (layer "B.Cu") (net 15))
 (segment (start 52.5272 54.25045) (end 53.34 53.43765) (width 0.8) (layer "B.Cu") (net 15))
 (segment (start 57.917 48.20025) (end 55.5852 48.20025) (width 0.8) (layer "B.Cu") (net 15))
 (segment (start 57.8612 48.25605) (end 57.917 48.20025) (width 0.8) (layer "B.Cu") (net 15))
 (segment (start 52.5272 56.52145) (end 52.5272 54.25045) (width 0.8) (layer "B.Cu") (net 15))
 (segment (start 57.8612 53.43765) (end 57.8612 48.25605) (width 0.8) (layer "B.Cu") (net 15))
 (segment (start 59.3344 56.57225) (end 59.3344 43.12025) (width 0.8) (layer "B.Cu") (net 3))
 (segment (start 56.5404 56.57225) (end 59.3344 56.57225) (width 0.8) (layer "B.Cu") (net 3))
 (segment (start 59.3344 43.12025) (end 55.5852 43.12025) (width 0.8) (layer "B.Cu") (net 3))
 (segment (start 22.7076 54.84505) (end 18.6028 50.74025) (width 0.8) (layer "B.Cu") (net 18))
 (segment (start 22.7076 56.43485) (end 22.7076 54.84505) (width 0.8) (layer "B.Cu") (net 18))
 (segment (start 16.3068 46.88445) (end 17.531 45.66025) (width 0.8) (layer "B.Cu") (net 20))
 (segment (start 16.3068 55.87605) (end 16.3068 46.88445) (width 0.8) (layer "B.Cu") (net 20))
 (segment (start 16.8506 56.41985) (end 16.3068 55.87605) (width 0.8) (layer "B.Cu") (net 20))
 (segment (start 18.5928 56.41985) (end 16.8506 56.41985) (width 0.8) (layer "B.Cu") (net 20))
 (segment (start 17.531 45.66025) (end 18.6028 45.66025) (width 0.8) (layer "B.Cu") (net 20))
 (segment (start 26.924 53.99645) (end 28.7528 52.16765) (width 0.8) (layer "B.Cu") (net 19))
 (segment (start 28.7528 52.16765) (end 28.7528 49.22125) (width 0.8) (layer "B.Cu") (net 19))
 (segment (start 27.7318 48.20025) (end 26.2228 48.20025) (width 0.8) (layer "B.Cu") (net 19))
 (segment (start 28.7528 49.22125) (end 27.7318 48.20025) (width 0.8) (layer "B.Cu") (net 19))
 (segment (start 26.924 56.48565) (end 26.924 53.99645) (width 0.8) (layer "B.Cu") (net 19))
 (segment (start 30.988 56.47065) (end 33.528 56.47065) (width 0.8) (layer "B.Cu") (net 21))
 (segment (start 28.8036 43.32845) (end 28.5954 43.12025) (width 0.8) (layer "B.Cu") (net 21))
 (segment (start 28.5954 43.12025) (end 26.2228 43.12025) (width 0.8) (layer "B.Cu") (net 21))
 (segment (start 28.8036 45.05565) (end 28.8036 43.32845) (width 0.8) (layer "B.Cu") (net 21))
 (segment (start 33.528 49.78005) (end 28.8036 45.05565) (width 0.8) (layer "B.Cu") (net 21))
 (segment (start 33.528 56.47065) (end 33.528 49.78005) (width 0.8) (layer "B.Cu") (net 21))
 (segment (start 31.9024 53.99645) (end 30.988 53.08205) (width 0.8) (layer "F.Cu") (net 12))
 (segment (start 37.5412 55.36805) (end 36.1696 53.99645) (width 0.8) (layer "F.Cu") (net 12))
 (segment (start 37.9476 52.42165) (end 44.2976 52.42165) (width 0.8) (layer "F.Cu") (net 12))
 (segment (start 37.6428 52.72645) (end 37.9476 52.42165) (width 0.8) (layer "F.Cu") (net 12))
 (segment (start 36.1696 53.99645) (end 31.9024 53.99645) (width 0.8) (layer "F.Cu") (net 12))
 (segment (start 44.2976 52.42165) (end 44.3992 52.32005) (width 0.8) (layer "F.Cu") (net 12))
 (via (at 44.3992 52.32005) (size 1.8) (drill 1) (layers "F.Cu" "B.Cu") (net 12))
 (via (at 30.988 53.08205) (size 1.8) (drill 1) (layers "F.Cu" "B.Cu") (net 12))
 (via (at 37.5412 55.36805) (size 1.8) (drill 1) (layers "F.Cu" "B.Cu") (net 12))
 (via (at 37.6428 52.72645) (size 1.8) (drill 1) (layers "F.Cu" "B.Cu") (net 12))
 (segment (start 22.1946 48.20025) (end 22.2504 48.25605) (width 1) (layer "B.Cu") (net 12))
 (segment (start 22.5552 45.66525) (end 22.5502 45.66025) (width 1) (layer "B.Cu") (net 12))
 (segment (start 18.6028 48.20025) (end 22.1946 48.20025) (width 1) (layer "B.Cu") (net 12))
 (segment (start 30.988 53.08205) (end 30.988 49.42445) (width 0.8) (layer "B.Cu") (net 12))
 (segment (start 27.2238 45.66025) (end 26.2228 45.66025) (width 0.8) (layer "B.Cu") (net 12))
 (segment (start 51.9734 50.74025) (end 51.5062 50.27305) (width 1) (layer "B.Cu") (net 12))
 (segment (start 47.9652 43.12025) (end 51.5062 43.12025) (width 1) (layer "B.Cu") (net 12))
 (segment (start 47.9652 48.20025) (end 51.4046 48.20025) (width 1) (layer "B.Cu") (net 12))
 (segment (start 37.6428 52.72645) (end 37.6428 55.26645) (width 0.8) (layer "B.Cu") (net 12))
 (segment (start 22.5552 50.74025) (end 22.5552 45.66525) (width 1) (layer "B.Cu") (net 12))
 (segment (start 51.5062 50.27305) (end 51.5062 48.30185) (width 1) (layer "B.Cu") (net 12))
 (segment (start 44.3026 48.20025) (end 47.9652 48.20025) (width 0.8) (layer "B.Cu") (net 12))
 (segment (start 51.5062 45.66025) (end 55.5852 45.66025) (width 1) (layer "B.Cu") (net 12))
 (segment (start 51.5062 43.12025) (end 51.5062 45.66025) (width 1) (layer "B.Cu") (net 12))
 (segment (start 30.988 49.42445) (end 27.2238 45.66025) (width 0.8) (layer "B.Cu") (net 12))
 (segment (start 44.3992 52.32005) (end 44.2976 52.21845) (width 0.8) (layer "B.Cu") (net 12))
 (segment (start 51.4046 48.20025) (end 51.5062 48.30185) (width 1) (layer "B.Cu") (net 12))
 (segment (start 44.2976 52.21845) (end 44.2976 48.20525) (width 0.8) (layer "B.Cu") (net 12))
 (segment (start 26.2228 50.74025) (end 22.5552 50.74025) (width 1) (layer "B.Cu") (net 12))
 (segment (start 22.5502 43.12025) (end 18.6028 43.12025) (width 1) (layer "B.Cu") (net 12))
 (segment (start 22.5502 45.66025) (end 22.5502 43.12025) (width 1) (layer "B.Cu") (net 12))
 (segment (start 44.2976 48.20525) (end 44.3026 48.20025) (width 0.8) (layer "B.Cu") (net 12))
 (segment (start 55.5852 50.74025) (end 51.9734 50.74025) (width 1) (layer "B.Cu") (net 12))
 (segment (start 51.5062 48.30185) (end 51.5062 43.12025) (width 1) (layer "B.Cu") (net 12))
 (segment (start 26.2228 45.66025) (end 22.5502 45.66025) (width 1) (layer "B.Cu") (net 12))
 (segment (start 37.6428 55.26645) (end 37.5412 55.36805) (width 0.8) (layer "B.Cu") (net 12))
 (segment (start 22.2504 48.25605) (end 22.5502 47.95625) (width 1) (layer "B.Cu") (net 12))
 (segment (start 22.5502 47.95625) (end 22.5502 45.66025) (width 1) (layer "B.Cu") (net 12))
 (segment (start 37.6428 52.72645) (end 37.6428 47.13845) (width 0.8) (layer "B.Cu") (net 12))
 (segment (start 47.9473 27.58835) (end 49.53 26.00565) (width 1) (layer "B.Cu") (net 17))
 (segment (start 55.5852 30.05965) (end 57.2516 28.39325) (width 1) (layer "B.Cu") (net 17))
 (segment (start 43.18 27.58835) (end 47.9473 27.58835) (width 1) (layer "B.Cu") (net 17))
 (segment (start 55.5852 30.68925) (end 55.5852 30.05965) (width 1) (layer "B.Cu") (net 17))
 (segment (start 49.53 26.00565) (end 55.2196 26.00565) (width 1) (layer "B.Cu") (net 17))
 (segment (start 55.2196 26.00565) (end 55.5852 26.37125) (width 1) (layer "B.Cu") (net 17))
 (segment (start 57.2516 28.39325) (end 60.6552 28.39325) (width 1) (layer "B.Cu") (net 17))
 (segment (start 55.5852 35.50025) (end 55.5852 30.68925) (width 1) (layer "B.Cu") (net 17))
 (segment (start 55.5852 26.37125) (end 55.5852 30.68925) (width 1) (layer "B.Cu") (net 17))
 (segment (start 55.5852 38.04025) (end 58.5166 38.04025) (width 1) (layer "B.Cu") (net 16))
 (segment (start 62.3316 24.07525) (end 63.0428 24.78645) (width 1) (layer "B.Cu") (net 16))
 (segment (start 40.7924 25.65005) (end 47.1424 25.65005) (width 1) (layer "B.Cu") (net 16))
 (segment (start 40.64 25.80245) (end 40.7924 25.65005) (width 1) (layer "B.Cu") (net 16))
 (segment (start 63.0428 31.18725) (end 62.5348 31.69525) (width 1) (layer "B.Cu") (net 16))
 (segment (start 62.5348 31.69525) (end 60.6552 31.69525) (width 1) (layer "B.Cu") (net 16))
 (segment (start 48.7172 24.07525) (end 62.3316 24.07525) (width 1) (layer "B.Cu") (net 16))
 (segment (start 58.6232 37.93365) (end 58.6232 31.64445) (width 1) (layer "B.Cu") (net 16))
 (segment (start 58.674 31.69525) (end 60.6552 31.69525) (width 1) (layer "B.Cu") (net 16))
 (segment (start 58.6232 31.64445) (end 58.674 31.69525) (width 1) (layer "B.Cu") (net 16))
 (segment (start 40.64 27.58835) (end 40.64 25.80245) (width 1) (layer "B.Cu") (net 16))
 (segment (start 58.5166 38.04025) (end 58.6232 37.93365) (width 1) (layer "B.Cu") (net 16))
 (segment (start 63.0428 24.78645) (end 63.0428 31.18725) (width 1) (layer "B.Cu") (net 16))
 (segment (start 47.1424 25.65005) (end 48.7172 24.07525) (width 1) (layer "B.Cu") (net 16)))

